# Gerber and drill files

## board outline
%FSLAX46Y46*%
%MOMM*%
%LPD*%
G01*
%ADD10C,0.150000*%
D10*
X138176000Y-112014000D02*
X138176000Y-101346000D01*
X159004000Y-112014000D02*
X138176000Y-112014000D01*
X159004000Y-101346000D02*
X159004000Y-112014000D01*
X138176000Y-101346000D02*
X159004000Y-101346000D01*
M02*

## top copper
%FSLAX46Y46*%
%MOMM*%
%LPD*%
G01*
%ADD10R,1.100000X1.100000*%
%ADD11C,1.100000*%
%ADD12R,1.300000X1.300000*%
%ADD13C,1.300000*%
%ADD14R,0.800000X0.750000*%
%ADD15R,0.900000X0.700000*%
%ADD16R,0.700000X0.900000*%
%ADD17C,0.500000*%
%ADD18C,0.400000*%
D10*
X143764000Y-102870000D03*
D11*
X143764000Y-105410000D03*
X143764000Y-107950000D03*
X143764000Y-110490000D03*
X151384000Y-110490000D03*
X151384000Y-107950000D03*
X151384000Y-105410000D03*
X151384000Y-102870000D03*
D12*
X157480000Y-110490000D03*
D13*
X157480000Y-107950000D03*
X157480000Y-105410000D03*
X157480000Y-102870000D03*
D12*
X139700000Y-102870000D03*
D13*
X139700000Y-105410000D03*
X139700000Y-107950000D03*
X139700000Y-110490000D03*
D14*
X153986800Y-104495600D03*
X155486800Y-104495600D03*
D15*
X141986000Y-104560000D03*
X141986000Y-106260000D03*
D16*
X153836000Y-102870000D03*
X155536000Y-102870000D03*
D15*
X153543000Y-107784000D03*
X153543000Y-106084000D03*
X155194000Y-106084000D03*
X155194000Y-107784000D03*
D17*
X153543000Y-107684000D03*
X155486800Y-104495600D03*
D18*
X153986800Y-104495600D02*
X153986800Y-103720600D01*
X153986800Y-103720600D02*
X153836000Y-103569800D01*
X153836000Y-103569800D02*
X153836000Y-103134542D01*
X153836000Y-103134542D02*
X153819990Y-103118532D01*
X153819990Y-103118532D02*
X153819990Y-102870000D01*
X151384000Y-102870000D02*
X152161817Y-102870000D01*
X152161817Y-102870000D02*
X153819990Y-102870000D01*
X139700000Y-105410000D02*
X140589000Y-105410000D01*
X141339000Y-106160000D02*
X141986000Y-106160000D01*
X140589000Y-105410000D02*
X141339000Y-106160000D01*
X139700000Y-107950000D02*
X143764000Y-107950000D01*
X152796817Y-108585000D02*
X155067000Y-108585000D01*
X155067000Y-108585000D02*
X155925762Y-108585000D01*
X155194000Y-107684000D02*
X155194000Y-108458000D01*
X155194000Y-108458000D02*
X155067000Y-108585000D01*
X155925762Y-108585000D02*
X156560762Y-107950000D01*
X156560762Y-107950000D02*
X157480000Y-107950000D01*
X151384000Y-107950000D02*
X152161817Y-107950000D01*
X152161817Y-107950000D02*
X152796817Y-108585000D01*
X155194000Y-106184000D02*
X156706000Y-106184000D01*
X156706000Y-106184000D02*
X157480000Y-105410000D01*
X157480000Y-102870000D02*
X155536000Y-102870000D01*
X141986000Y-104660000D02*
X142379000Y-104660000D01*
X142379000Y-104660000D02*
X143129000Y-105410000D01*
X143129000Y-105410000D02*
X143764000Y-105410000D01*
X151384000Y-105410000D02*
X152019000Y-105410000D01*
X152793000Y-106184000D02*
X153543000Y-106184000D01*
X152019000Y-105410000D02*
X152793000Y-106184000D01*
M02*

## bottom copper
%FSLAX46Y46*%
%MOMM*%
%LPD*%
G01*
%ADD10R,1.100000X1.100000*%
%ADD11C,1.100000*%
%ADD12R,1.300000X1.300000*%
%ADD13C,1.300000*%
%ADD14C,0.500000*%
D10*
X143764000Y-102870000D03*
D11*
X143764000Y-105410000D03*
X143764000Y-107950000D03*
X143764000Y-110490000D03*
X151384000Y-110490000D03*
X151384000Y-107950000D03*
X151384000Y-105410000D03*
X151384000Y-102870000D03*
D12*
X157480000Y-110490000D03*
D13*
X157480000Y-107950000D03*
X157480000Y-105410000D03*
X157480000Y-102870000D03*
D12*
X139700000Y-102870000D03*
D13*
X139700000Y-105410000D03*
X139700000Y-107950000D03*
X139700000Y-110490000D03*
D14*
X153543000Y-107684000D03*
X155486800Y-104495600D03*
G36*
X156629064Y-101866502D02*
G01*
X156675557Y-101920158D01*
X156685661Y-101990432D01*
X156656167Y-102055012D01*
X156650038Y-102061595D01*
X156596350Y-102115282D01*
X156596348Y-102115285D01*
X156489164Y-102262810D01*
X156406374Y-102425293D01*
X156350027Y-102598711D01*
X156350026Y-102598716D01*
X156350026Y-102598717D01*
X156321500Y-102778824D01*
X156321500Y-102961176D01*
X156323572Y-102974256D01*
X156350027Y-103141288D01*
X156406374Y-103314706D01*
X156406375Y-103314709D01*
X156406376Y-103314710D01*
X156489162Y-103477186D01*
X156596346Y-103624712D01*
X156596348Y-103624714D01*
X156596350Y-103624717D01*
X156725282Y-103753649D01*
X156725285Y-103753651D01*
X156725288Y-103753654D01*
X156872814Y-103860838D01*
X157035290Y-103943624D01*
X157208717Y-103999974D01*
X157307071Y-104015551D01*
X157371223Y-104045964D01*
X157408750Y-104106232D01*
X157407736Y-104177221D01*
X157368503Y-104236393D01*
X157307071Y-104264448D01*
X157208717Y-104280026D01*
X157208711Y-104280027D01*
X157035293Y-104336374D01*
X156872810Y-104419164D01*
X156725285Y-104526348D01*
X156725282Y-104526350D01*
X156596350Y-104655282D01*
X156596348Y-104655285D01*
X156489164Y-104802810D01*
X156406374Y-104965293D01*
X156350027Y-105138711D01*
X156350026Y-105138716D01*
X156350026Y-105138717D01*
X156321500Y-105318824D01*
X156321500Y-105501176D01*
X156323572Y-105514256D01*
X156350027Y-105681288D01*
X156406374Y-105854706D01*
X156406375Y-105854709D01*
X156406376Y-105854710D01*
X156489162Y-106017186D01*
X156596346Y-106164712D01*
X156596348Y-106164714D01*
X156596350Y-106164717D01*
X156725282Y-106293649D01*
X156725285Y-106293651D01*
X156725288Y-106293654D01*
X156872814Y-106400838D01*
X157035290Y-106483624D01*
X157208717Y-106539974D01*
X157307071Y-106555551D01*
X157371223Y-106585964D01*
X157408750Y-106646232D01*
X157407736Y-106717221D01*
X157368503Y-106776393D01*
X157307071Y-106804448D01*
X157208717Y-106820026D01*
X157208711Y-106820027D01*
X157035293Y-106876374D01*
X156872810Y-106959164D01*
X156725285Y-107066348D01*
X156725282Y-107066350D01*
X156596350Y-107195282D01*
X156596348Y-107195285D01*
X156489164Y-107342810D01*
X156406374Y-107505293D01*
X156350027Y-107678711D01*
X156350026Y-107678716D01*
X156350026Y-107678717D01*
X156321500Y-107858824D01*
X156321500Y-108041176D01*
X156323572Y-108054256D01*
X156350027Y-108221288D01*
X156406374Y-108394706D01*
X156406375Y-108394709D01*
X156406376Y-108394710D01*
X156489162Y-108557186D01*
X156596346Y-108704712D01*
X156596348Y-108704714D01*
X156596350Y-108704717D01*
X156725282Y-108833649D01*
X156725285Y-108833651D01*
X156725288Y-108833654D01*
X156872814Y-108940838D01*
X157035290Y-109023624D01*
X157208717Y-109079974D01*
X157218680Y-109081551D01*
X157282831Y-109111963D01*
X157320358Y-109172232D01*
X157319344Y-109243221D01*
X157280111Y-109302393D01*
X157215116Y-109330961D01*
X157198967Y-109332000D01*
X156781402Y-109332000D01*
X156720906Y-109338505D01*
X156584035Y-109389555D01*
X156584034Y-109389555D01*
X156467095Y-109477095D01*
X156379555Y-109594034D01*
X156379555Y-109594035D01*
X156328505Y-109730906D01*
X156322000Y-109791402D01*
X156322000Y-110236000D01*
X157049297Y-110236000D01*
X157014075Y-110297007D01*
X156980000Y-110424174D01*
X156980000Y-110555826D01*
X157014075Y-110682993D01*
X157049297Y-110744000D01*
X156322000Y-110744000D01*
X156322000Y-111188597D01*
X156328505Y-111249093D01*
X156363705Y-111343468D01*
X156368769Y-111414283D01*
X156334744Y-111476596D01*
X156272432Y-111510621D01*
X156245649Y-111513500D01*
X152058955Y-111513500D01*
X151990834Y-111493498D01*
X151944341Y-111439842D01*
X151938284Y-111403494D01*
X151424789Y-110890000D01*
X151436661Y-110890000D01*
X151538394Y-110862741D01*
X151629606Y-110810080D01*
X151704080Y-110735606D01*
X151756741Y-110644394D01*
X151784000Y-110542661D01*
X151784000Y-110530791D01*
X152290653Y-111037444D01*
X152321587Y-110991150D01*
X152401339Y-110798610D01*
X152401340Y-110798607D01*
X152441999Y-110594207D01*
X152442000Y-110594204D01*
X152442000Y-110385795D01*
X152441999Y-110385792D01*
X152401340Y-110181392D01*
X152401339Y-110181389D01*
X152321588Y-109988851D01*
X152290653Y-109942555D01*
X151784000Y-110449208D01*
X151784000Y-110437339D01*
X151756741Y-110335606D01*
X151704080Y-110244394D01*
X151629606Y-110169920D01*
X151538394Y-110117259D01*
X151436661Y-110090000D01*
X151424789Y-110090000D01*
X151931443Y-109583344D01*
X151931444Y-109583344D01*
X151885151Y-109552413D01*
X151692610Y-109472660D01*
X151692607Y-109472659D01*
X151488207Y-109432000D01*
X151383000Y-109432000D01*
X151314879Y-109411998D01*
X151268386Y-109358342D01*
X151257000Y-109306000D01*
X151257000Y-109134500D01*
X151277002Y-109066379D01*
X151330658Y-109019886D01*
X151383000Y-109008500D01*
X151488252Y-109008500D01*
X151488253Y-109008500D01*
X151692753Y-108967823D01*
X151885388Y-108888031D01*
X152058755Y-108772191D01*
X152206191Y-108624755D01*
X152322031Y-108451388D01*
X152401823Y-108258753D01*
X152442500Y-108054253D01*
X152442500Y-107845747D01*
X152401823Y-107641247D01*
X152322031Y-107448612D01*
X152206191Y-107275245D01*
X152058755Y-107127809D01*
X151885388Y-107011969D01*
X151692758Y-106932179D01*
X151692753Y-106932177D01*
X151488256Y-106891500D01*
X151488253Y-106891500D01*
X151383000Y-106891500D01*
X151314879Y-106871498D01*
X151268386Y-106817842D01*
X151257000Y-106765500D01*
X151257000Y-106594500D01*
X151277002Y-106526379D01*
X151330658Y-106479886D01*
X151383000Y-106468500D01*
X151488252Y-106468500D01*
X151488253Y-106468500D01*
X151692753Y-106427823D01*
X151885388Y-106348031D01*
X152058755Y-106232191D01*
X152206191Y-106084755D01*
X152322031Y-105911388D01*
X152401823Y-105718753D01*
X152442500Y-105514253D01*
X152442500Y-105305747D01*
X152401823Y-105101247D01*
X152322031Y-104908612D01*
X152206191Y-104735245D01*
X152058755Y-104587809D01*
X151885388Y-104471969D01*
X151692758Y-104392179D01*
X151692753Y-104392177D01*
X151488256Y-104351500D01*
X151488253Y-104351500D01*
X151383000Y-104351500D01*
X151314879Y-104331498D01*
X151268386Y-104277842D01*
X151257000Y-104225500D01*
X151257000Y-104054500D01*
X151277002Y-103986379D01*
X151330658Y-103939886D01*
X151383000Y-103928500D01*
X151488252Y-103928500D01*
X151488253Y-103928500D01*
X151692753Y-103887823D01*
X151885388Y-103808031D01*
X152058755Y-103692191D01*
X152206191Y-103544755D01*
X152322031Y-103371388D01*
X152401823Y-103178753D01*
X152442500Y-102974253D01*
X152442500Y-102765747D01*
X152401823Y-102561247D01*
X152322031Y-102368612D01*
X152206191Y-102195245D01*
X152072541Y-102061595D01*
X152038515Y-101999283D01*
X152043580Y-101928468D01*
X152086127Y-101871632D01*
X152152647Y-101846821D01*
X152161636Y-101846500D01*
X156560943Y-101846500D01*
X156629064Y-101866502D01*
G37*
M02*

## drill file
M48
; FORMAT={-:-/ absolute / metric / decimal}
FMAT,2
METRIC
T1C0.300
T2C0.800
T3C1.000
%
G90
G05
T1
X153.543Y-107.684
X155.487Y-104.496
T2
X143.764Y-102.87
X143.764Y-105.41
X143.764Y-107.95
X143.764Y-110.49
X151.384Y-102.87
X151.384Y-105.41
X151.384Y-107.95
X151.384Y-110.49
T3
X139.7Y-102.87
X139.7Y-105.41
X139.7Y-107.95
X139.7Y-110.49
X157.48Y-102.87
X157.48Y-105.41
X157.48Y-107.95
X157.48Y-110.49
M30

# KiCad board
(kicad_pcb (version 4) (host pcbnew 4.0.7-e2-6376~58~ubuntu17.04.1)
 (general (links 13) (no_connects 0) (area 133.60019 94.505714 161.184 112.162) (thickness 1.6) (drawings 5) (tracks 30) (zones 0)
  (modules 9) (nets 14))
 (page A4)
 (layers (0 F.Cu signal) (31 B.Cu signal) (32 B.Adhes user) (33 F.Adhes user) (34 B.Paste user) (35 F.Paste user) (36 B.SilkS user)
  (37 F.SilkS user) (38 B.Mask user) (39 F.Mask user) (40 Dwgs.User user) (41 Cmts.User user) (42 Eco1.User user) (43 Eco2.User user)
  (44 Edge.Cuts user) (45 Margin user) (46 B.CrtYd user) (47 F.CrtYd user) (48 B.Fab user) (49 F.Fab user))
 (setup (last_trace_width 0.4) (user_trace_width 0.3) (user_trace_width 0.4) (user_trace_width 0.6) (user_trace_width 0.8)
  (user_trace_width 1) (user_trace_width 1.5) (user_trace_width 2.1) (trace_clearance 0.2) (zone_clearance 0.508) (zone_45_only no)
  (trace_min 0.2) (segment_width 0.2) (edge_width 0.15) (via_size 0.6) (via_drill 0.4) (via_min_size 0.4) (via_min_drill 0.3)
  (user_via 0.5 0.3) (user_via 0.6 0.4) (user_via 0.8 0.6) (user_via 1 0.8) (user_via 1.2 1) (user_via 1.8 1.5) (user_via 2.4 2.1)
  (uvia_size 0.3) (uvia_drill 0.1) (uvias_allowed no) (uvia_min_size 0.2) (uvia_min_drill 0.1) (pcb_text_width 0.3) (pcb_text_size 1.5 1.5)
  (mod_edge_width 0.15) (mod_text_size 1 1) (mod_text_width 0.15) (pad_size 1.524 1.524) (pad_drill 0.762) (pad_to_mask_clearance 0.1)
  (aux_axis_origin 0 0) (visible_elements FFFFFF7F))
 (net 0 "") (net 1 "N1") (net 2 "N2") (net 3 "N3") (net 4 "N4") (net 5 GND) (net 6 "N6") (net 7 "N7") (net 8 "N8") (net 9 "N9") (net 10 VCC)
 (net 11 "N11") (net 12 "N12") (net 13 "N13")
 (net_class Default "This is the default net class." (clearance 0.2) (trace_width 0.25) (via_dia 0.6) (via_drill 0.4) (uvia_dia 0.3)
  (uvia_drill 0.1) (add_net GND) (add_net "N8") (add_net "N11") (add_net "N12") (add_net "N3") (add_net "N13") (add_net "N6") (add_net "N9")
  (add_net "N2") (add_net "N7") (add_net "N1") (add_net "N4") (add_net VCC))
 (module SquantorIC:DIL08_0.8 (layer F.Cu) (at 147.574 106.68 270)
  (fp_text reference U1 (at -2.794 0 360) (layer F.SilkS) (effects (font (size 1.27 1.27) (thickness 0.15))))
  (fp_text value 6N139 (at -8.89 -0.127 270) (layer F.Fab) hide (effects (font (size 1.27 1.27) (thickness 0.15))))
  (pad 1 thru_hole rect (at -3.81 3.81 90) (size 1.1 1.1) (drill 0.8) (layers *.Cu *.Paste *.SilkS *.Mask) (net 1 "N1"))
  (pad 2 thru_hole circle (at -1.27 3.81 90) (size 1.1 1.1) (drill 0.8) (layers *.Cu *.Paste *.SilkS *.Mask) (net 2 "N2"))
  (pad 3 thru_hole circle (at 1.27 3.81 90) (size 1.1 1.1) (drill 0.8) (layers *.Cu *.Paste *.SilkS *.Mask) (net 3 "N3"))
  (pad 4 thru_hole circle (at 3.81 3.81 90) (size 1.1 1.1) (drill 0.8) (layers *.Cu *.Paste *.SilkS *.Mask) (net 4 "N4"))
  (pad 5 thru_hole circle (at 3.81 -3.81 90) (size 1.1 1.1) (drill 0.8) (layers *.Cu *.Paste *.SilkS *.Mask) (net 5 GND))
  (pad 6 thru_hole circle (at 1.27 -3.81 90) (size 1.1 1.1) (drill 0.8) (layers *.Cu *.Paste *.SilkS *.Mask) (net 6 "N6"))
  (pad 7 thru_hole circle (at -1.27 -3.81 90) (size 1.1 1.1) (drill 0.8) (layers *.Cu *.Paste *.SilkS *.Mask) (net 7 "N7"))
  (pad 8 thru_hole circle (at -3.81 -3.81 90) (size 1.1 1.1) (drill 0.8) (layers *.Cu *.Paste *.SilkS *.Mask) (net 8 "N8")))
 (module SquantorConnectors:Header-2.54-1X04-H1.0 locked (layer B.Cu) (at 157.48 106.68 90)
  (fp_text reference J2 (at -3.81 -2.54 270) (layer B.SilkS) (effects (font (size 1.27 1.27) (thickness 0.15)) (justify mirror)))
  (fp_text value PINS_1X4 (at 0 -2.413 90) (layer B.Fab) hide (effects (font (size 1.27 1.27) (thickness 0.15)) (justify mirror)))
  (pad 1 thru_hole rect (at -3.81 0 270) (size 1.3 1.3) (drill 1) (layers *.Cu *.Paste *.SilkS *.Mask) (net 5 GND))
  (pad 2 thru_hole circle (at -1.27 0 270) (size 1.3 1.3) (drill 1) (layers *.Cu *.Paste *.SilkS *.Mask) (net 6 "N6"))
  (pad 3 thru_hole circle (at 1.27 0 270) (size 1.3 1.3) (drill 1) (layers *.Cu *.Paste *.SilkS *.Mask) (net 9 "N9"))
  (pad 4 thru_hole circle (at 3.81 0 270) (size 1.3 1.3) (drill 1) (layers *.Cu *.Paste *.SilkS *.Mask) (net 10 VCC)))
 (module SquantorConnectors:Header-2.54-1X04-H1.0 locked (layer B.Cu) (at 139.7 106.68 270)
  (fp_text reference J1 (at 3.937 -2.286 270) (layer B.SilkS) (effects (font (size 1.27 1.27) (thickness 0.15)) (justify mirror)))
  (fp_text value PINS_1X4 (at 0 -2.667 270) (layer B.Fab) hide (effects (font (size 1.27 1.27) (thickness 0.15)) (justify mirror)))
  (pad 1 thru_hole rect (at -3.81 0 90) (size 1.3 1.3) (drill 1) (layers *.Cu *.Paste *.SilkS *.Mask) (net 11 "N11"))
  (pad 2 thru_hole circle (at -1.27 0 90) (size 1.3 1.3) (drill 1) (layers *.Cu *.Paste *.SilkS *.Mask) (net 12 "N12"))
  (pad 3 thru_hole circle (at 1.27 0 90) (size 1.3 1.3) (drill 1) (layers *.Cu *.Paste *.SilkS *.Mask) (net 3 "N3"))
  (pad 4 thru_hole circle (at 3.81 0 90) (size 1.3 1.3) (drill 1) (layers *.Cu *.Paste *.SilkS *.Mask) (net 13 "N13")))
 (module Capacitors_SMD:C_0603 (layer F.Cu) (at 154.7368 104.4956)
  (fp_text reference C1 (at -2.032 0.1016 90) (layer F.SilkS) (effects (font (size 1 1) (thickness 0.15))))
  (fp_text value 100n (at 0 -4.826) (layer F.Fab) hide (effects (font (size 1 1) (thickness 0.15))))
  (pad 1 smd rect (at -0.75 0) (size 0.8 0.75) (layers F.Cu F.Paste F.Mask) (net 8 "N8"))
  (pad 2 smd rect (at 0.75 0) (size 0.8 0.75) (layers F.Cu F.Paste F.Mask) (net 5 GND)))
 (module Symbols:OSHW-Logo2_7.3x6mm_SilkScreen (layer B.Cu) (at 147.574 104.521 180)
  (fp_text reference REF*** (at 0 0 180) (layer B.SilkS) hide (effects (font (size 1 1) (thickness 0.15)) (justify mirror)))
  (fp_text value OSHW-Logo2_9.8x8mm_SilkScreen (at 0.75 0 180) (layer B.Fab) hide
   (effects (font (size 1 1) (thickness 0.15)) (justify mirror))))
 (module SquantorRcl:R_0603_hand (layer F.Cu) (at 141.986 105.41 270)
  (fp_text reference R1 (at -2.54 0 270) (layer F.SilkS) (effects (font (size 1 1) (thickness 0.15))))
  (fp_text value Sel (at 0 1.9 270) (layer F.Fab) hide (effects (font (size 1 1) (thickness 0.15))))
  (pad 1 smd rect (at -0.85 0 270) (size 0.7 0.9) (layers F.Cu F.Paste F.Mask) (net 2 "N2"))
  (pad 2 smd rect (at 0.85 0 270) (size 0.7 0.9) (layers F.Cu F.Paste F.Mask) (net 12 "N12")))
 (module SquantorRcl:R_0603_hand (layer F.Cu) (at 154.686 102.87)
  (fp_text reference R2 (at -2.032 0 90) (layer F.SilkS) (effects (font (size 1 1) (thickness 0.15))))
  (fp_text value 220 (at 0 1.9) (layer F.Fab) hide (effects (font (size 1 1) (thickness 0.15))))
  (pad 1 smd rect (at -0.85 0) (size 0.7 0.9) (layers F.Cu F.Paste F.Mask) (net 8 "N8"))
  (pad 2 smd rect (at 0.85 0) (size 0.7 0.9) (layers F.Cu F.Paste F.Mask) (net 10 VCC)))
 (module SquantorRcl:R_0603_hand (layer F.Cu) (at 153.543 106.934 90)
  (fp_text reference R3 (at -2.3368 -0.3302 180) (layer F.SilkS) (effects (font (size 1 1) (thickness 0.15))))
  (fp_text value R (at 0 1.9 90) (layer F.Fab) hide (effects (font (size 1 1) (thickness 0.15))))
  (pad 1 smd rect (at -0.85 0 90) (size 0.7 0.9) (layers F.Cu F.Paste F.Mask) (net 5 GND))
  (pad 2 smd rect (at 0.85 0 90) (size 0.7 0.9) (layers F.Cu F.Paste F.Mask) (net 7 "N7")))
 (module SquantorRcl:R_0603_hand (layer F.Cu) (at 155.194 106.934 270)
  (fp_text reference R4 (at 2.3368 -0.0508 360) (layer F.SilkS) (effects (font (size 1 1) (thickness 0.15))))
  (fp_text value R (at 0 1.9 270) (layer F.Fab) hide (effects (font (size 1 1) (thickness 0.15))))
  (pad 1 smd rect (at -0.85 0 270) (size 0.7 0.9) (layers F.Cu F.Paste F.Mask) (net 9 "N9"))
  (pad 2 smd rect (at 0.85 0 270) (size 0.7 0.9) (layers F.Cu F.Paste F.Mask) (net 6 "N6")))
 (gr_line (start 138.176 112.014) (end 138.176 101.346) (angle 90) (layer Edge.Cuts) (width 0.15))
 (gr_line (start 159.004 112.014) (end 138.176 112.014) (angle 90) (layer Edge.Cuts) (width 0.15))
 (gr_line (start 159.004 101.346) (end 159.004 112.014) (angle 90) (layer Edge.Cuts) (width 0.15))
 (gr_line (start 138.176 101.346) (end 159.004 101.346) (angle 90) (layer Edge.Cuts) (width 0.15))
 (segment (start 153.9868 104.4956) (end 153.9868 103.7206) (width 0.4) (layer F.Cu) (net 8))
 (segment (start 153.9868 103.7206) (end 153.836 103.5698) (width 0.4) (layer F.Cu) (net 8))
 (segment (start 153.836 103.5698) (end 153.836 103.134542) (width 0.4) (layer F.Cu) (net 8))
 (segment (start 153.836 103.134542) (end 153.81999 103.118532) (width 0.4) (layer F.Cu) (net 8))
 (segment (start 153.81999 103.118532) (end 153.81999 102.87) (width 0.4) (layer F.Cu) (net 8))
 (segment (start 151.384 102.87) (end 152.161817 102.87) (width 0.4) (layer F.Cu) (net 8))
 (segment (start 152.161817 102.87) (end 153.81999 102.87) (width 0.4) (layer F.Cu) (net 8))
 (via (at 153.543 107.684) (size 0.5) (drill 0.3) (layers F.Cu B.Cu) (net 5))
 (via (at 155.4868 104.4956) (size 0.5) (drill 0.3) (layers F.Cu B.Cu) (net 5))
 (segment (start 139.7 105.41) (end 140.589 105.41) (width 0.4) (layer F.Cu) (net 12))
 (segment (start 141.339 106.16) (end 141.986 106.16) (width 0.4) (layer F.Cu) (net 12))
 (segment (start 140.589 105.41) (end 141.339 106.16) (width 0.4) (layer F.Cu) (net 12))
 (segment (start 139.7 107.95) (end 143.764 107.95) (width 0.4) (layer F.Cu) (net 3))
 (segment (start 152.796817 108.585) (end 155.067 108.585) (width 0.4) (layer F.Cu) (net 6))
 (segment (start 155.067 108.585) (end 155.925762 108.585) (width 0.4) (layer F.Cu) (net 6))
 (segment (start 155.194 107.684) (end 155.194 108.458) (width 0.4) (layer F.Cu) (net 6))
 (segment (start 155.194 108.458) (end 155.067 108.585) (width 0.4) (layer F.Cu) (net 6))
 (segment (start 155.925762 108.585) (end 156.560762 107.95) (width 0.4) (layer F.Cu) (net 6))
 (segment (start 156.560762 107.95) (end 157.48 107.95) (width 0.4) (layer F.Cu) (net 6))
 (segment (start 151.384 107.95) (end 152.161817 107.95) (width 0.4) (layer F.Cu) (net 6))
 (segment (start 152.161817 107.95) (end 152.796817 108.585) (width 0.4) (layer F.Cu) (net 6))
 (segment (start 155.194 106.184) (end 156.706 106.184) (width 0.4) (layer F.Cu) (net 9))
 (segment (start 156.706 106.184) (end 157.48 105.41) (width 0.4) (layer F.Cu) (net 9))
 (segment (start 157.48 102.87) (end 155.536 102.87) (width 0.4) (layer F.Cu) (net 10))
 (segment (start 141.986 104.66) (end 142.379 104.66) (width 0.4) (layer F.Cu) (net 2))
 (segment (start 142.379 104.66) (end 143.129 105.41) (width 0.4) (layer F.Cu) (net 2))
 (segment (start 143.129 105.41) (end 143.764 105.41) (width 0.4) (layer F.Cu) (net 2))
 (segment (start 151.384 105.41) (end 152.019 105.41) (width 0.4) (layer F.Cu) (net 7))
 (segment (start 152.793 106.184) (end 153.543 106.184) (width 0.4) (layer F.Cu) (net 7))
 (segment (start 152.019 105.41) (end 152.793 106.184) (width 0.4) (layer F.Cu) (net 7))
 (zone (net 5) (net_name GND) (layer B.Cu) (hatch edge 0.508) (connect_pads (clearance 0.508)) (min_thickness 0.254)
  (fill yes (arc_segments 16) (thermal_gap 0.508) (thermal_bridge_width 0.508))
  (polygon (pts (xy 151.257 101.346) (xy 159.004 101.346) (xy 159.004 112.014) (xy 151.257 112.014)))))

